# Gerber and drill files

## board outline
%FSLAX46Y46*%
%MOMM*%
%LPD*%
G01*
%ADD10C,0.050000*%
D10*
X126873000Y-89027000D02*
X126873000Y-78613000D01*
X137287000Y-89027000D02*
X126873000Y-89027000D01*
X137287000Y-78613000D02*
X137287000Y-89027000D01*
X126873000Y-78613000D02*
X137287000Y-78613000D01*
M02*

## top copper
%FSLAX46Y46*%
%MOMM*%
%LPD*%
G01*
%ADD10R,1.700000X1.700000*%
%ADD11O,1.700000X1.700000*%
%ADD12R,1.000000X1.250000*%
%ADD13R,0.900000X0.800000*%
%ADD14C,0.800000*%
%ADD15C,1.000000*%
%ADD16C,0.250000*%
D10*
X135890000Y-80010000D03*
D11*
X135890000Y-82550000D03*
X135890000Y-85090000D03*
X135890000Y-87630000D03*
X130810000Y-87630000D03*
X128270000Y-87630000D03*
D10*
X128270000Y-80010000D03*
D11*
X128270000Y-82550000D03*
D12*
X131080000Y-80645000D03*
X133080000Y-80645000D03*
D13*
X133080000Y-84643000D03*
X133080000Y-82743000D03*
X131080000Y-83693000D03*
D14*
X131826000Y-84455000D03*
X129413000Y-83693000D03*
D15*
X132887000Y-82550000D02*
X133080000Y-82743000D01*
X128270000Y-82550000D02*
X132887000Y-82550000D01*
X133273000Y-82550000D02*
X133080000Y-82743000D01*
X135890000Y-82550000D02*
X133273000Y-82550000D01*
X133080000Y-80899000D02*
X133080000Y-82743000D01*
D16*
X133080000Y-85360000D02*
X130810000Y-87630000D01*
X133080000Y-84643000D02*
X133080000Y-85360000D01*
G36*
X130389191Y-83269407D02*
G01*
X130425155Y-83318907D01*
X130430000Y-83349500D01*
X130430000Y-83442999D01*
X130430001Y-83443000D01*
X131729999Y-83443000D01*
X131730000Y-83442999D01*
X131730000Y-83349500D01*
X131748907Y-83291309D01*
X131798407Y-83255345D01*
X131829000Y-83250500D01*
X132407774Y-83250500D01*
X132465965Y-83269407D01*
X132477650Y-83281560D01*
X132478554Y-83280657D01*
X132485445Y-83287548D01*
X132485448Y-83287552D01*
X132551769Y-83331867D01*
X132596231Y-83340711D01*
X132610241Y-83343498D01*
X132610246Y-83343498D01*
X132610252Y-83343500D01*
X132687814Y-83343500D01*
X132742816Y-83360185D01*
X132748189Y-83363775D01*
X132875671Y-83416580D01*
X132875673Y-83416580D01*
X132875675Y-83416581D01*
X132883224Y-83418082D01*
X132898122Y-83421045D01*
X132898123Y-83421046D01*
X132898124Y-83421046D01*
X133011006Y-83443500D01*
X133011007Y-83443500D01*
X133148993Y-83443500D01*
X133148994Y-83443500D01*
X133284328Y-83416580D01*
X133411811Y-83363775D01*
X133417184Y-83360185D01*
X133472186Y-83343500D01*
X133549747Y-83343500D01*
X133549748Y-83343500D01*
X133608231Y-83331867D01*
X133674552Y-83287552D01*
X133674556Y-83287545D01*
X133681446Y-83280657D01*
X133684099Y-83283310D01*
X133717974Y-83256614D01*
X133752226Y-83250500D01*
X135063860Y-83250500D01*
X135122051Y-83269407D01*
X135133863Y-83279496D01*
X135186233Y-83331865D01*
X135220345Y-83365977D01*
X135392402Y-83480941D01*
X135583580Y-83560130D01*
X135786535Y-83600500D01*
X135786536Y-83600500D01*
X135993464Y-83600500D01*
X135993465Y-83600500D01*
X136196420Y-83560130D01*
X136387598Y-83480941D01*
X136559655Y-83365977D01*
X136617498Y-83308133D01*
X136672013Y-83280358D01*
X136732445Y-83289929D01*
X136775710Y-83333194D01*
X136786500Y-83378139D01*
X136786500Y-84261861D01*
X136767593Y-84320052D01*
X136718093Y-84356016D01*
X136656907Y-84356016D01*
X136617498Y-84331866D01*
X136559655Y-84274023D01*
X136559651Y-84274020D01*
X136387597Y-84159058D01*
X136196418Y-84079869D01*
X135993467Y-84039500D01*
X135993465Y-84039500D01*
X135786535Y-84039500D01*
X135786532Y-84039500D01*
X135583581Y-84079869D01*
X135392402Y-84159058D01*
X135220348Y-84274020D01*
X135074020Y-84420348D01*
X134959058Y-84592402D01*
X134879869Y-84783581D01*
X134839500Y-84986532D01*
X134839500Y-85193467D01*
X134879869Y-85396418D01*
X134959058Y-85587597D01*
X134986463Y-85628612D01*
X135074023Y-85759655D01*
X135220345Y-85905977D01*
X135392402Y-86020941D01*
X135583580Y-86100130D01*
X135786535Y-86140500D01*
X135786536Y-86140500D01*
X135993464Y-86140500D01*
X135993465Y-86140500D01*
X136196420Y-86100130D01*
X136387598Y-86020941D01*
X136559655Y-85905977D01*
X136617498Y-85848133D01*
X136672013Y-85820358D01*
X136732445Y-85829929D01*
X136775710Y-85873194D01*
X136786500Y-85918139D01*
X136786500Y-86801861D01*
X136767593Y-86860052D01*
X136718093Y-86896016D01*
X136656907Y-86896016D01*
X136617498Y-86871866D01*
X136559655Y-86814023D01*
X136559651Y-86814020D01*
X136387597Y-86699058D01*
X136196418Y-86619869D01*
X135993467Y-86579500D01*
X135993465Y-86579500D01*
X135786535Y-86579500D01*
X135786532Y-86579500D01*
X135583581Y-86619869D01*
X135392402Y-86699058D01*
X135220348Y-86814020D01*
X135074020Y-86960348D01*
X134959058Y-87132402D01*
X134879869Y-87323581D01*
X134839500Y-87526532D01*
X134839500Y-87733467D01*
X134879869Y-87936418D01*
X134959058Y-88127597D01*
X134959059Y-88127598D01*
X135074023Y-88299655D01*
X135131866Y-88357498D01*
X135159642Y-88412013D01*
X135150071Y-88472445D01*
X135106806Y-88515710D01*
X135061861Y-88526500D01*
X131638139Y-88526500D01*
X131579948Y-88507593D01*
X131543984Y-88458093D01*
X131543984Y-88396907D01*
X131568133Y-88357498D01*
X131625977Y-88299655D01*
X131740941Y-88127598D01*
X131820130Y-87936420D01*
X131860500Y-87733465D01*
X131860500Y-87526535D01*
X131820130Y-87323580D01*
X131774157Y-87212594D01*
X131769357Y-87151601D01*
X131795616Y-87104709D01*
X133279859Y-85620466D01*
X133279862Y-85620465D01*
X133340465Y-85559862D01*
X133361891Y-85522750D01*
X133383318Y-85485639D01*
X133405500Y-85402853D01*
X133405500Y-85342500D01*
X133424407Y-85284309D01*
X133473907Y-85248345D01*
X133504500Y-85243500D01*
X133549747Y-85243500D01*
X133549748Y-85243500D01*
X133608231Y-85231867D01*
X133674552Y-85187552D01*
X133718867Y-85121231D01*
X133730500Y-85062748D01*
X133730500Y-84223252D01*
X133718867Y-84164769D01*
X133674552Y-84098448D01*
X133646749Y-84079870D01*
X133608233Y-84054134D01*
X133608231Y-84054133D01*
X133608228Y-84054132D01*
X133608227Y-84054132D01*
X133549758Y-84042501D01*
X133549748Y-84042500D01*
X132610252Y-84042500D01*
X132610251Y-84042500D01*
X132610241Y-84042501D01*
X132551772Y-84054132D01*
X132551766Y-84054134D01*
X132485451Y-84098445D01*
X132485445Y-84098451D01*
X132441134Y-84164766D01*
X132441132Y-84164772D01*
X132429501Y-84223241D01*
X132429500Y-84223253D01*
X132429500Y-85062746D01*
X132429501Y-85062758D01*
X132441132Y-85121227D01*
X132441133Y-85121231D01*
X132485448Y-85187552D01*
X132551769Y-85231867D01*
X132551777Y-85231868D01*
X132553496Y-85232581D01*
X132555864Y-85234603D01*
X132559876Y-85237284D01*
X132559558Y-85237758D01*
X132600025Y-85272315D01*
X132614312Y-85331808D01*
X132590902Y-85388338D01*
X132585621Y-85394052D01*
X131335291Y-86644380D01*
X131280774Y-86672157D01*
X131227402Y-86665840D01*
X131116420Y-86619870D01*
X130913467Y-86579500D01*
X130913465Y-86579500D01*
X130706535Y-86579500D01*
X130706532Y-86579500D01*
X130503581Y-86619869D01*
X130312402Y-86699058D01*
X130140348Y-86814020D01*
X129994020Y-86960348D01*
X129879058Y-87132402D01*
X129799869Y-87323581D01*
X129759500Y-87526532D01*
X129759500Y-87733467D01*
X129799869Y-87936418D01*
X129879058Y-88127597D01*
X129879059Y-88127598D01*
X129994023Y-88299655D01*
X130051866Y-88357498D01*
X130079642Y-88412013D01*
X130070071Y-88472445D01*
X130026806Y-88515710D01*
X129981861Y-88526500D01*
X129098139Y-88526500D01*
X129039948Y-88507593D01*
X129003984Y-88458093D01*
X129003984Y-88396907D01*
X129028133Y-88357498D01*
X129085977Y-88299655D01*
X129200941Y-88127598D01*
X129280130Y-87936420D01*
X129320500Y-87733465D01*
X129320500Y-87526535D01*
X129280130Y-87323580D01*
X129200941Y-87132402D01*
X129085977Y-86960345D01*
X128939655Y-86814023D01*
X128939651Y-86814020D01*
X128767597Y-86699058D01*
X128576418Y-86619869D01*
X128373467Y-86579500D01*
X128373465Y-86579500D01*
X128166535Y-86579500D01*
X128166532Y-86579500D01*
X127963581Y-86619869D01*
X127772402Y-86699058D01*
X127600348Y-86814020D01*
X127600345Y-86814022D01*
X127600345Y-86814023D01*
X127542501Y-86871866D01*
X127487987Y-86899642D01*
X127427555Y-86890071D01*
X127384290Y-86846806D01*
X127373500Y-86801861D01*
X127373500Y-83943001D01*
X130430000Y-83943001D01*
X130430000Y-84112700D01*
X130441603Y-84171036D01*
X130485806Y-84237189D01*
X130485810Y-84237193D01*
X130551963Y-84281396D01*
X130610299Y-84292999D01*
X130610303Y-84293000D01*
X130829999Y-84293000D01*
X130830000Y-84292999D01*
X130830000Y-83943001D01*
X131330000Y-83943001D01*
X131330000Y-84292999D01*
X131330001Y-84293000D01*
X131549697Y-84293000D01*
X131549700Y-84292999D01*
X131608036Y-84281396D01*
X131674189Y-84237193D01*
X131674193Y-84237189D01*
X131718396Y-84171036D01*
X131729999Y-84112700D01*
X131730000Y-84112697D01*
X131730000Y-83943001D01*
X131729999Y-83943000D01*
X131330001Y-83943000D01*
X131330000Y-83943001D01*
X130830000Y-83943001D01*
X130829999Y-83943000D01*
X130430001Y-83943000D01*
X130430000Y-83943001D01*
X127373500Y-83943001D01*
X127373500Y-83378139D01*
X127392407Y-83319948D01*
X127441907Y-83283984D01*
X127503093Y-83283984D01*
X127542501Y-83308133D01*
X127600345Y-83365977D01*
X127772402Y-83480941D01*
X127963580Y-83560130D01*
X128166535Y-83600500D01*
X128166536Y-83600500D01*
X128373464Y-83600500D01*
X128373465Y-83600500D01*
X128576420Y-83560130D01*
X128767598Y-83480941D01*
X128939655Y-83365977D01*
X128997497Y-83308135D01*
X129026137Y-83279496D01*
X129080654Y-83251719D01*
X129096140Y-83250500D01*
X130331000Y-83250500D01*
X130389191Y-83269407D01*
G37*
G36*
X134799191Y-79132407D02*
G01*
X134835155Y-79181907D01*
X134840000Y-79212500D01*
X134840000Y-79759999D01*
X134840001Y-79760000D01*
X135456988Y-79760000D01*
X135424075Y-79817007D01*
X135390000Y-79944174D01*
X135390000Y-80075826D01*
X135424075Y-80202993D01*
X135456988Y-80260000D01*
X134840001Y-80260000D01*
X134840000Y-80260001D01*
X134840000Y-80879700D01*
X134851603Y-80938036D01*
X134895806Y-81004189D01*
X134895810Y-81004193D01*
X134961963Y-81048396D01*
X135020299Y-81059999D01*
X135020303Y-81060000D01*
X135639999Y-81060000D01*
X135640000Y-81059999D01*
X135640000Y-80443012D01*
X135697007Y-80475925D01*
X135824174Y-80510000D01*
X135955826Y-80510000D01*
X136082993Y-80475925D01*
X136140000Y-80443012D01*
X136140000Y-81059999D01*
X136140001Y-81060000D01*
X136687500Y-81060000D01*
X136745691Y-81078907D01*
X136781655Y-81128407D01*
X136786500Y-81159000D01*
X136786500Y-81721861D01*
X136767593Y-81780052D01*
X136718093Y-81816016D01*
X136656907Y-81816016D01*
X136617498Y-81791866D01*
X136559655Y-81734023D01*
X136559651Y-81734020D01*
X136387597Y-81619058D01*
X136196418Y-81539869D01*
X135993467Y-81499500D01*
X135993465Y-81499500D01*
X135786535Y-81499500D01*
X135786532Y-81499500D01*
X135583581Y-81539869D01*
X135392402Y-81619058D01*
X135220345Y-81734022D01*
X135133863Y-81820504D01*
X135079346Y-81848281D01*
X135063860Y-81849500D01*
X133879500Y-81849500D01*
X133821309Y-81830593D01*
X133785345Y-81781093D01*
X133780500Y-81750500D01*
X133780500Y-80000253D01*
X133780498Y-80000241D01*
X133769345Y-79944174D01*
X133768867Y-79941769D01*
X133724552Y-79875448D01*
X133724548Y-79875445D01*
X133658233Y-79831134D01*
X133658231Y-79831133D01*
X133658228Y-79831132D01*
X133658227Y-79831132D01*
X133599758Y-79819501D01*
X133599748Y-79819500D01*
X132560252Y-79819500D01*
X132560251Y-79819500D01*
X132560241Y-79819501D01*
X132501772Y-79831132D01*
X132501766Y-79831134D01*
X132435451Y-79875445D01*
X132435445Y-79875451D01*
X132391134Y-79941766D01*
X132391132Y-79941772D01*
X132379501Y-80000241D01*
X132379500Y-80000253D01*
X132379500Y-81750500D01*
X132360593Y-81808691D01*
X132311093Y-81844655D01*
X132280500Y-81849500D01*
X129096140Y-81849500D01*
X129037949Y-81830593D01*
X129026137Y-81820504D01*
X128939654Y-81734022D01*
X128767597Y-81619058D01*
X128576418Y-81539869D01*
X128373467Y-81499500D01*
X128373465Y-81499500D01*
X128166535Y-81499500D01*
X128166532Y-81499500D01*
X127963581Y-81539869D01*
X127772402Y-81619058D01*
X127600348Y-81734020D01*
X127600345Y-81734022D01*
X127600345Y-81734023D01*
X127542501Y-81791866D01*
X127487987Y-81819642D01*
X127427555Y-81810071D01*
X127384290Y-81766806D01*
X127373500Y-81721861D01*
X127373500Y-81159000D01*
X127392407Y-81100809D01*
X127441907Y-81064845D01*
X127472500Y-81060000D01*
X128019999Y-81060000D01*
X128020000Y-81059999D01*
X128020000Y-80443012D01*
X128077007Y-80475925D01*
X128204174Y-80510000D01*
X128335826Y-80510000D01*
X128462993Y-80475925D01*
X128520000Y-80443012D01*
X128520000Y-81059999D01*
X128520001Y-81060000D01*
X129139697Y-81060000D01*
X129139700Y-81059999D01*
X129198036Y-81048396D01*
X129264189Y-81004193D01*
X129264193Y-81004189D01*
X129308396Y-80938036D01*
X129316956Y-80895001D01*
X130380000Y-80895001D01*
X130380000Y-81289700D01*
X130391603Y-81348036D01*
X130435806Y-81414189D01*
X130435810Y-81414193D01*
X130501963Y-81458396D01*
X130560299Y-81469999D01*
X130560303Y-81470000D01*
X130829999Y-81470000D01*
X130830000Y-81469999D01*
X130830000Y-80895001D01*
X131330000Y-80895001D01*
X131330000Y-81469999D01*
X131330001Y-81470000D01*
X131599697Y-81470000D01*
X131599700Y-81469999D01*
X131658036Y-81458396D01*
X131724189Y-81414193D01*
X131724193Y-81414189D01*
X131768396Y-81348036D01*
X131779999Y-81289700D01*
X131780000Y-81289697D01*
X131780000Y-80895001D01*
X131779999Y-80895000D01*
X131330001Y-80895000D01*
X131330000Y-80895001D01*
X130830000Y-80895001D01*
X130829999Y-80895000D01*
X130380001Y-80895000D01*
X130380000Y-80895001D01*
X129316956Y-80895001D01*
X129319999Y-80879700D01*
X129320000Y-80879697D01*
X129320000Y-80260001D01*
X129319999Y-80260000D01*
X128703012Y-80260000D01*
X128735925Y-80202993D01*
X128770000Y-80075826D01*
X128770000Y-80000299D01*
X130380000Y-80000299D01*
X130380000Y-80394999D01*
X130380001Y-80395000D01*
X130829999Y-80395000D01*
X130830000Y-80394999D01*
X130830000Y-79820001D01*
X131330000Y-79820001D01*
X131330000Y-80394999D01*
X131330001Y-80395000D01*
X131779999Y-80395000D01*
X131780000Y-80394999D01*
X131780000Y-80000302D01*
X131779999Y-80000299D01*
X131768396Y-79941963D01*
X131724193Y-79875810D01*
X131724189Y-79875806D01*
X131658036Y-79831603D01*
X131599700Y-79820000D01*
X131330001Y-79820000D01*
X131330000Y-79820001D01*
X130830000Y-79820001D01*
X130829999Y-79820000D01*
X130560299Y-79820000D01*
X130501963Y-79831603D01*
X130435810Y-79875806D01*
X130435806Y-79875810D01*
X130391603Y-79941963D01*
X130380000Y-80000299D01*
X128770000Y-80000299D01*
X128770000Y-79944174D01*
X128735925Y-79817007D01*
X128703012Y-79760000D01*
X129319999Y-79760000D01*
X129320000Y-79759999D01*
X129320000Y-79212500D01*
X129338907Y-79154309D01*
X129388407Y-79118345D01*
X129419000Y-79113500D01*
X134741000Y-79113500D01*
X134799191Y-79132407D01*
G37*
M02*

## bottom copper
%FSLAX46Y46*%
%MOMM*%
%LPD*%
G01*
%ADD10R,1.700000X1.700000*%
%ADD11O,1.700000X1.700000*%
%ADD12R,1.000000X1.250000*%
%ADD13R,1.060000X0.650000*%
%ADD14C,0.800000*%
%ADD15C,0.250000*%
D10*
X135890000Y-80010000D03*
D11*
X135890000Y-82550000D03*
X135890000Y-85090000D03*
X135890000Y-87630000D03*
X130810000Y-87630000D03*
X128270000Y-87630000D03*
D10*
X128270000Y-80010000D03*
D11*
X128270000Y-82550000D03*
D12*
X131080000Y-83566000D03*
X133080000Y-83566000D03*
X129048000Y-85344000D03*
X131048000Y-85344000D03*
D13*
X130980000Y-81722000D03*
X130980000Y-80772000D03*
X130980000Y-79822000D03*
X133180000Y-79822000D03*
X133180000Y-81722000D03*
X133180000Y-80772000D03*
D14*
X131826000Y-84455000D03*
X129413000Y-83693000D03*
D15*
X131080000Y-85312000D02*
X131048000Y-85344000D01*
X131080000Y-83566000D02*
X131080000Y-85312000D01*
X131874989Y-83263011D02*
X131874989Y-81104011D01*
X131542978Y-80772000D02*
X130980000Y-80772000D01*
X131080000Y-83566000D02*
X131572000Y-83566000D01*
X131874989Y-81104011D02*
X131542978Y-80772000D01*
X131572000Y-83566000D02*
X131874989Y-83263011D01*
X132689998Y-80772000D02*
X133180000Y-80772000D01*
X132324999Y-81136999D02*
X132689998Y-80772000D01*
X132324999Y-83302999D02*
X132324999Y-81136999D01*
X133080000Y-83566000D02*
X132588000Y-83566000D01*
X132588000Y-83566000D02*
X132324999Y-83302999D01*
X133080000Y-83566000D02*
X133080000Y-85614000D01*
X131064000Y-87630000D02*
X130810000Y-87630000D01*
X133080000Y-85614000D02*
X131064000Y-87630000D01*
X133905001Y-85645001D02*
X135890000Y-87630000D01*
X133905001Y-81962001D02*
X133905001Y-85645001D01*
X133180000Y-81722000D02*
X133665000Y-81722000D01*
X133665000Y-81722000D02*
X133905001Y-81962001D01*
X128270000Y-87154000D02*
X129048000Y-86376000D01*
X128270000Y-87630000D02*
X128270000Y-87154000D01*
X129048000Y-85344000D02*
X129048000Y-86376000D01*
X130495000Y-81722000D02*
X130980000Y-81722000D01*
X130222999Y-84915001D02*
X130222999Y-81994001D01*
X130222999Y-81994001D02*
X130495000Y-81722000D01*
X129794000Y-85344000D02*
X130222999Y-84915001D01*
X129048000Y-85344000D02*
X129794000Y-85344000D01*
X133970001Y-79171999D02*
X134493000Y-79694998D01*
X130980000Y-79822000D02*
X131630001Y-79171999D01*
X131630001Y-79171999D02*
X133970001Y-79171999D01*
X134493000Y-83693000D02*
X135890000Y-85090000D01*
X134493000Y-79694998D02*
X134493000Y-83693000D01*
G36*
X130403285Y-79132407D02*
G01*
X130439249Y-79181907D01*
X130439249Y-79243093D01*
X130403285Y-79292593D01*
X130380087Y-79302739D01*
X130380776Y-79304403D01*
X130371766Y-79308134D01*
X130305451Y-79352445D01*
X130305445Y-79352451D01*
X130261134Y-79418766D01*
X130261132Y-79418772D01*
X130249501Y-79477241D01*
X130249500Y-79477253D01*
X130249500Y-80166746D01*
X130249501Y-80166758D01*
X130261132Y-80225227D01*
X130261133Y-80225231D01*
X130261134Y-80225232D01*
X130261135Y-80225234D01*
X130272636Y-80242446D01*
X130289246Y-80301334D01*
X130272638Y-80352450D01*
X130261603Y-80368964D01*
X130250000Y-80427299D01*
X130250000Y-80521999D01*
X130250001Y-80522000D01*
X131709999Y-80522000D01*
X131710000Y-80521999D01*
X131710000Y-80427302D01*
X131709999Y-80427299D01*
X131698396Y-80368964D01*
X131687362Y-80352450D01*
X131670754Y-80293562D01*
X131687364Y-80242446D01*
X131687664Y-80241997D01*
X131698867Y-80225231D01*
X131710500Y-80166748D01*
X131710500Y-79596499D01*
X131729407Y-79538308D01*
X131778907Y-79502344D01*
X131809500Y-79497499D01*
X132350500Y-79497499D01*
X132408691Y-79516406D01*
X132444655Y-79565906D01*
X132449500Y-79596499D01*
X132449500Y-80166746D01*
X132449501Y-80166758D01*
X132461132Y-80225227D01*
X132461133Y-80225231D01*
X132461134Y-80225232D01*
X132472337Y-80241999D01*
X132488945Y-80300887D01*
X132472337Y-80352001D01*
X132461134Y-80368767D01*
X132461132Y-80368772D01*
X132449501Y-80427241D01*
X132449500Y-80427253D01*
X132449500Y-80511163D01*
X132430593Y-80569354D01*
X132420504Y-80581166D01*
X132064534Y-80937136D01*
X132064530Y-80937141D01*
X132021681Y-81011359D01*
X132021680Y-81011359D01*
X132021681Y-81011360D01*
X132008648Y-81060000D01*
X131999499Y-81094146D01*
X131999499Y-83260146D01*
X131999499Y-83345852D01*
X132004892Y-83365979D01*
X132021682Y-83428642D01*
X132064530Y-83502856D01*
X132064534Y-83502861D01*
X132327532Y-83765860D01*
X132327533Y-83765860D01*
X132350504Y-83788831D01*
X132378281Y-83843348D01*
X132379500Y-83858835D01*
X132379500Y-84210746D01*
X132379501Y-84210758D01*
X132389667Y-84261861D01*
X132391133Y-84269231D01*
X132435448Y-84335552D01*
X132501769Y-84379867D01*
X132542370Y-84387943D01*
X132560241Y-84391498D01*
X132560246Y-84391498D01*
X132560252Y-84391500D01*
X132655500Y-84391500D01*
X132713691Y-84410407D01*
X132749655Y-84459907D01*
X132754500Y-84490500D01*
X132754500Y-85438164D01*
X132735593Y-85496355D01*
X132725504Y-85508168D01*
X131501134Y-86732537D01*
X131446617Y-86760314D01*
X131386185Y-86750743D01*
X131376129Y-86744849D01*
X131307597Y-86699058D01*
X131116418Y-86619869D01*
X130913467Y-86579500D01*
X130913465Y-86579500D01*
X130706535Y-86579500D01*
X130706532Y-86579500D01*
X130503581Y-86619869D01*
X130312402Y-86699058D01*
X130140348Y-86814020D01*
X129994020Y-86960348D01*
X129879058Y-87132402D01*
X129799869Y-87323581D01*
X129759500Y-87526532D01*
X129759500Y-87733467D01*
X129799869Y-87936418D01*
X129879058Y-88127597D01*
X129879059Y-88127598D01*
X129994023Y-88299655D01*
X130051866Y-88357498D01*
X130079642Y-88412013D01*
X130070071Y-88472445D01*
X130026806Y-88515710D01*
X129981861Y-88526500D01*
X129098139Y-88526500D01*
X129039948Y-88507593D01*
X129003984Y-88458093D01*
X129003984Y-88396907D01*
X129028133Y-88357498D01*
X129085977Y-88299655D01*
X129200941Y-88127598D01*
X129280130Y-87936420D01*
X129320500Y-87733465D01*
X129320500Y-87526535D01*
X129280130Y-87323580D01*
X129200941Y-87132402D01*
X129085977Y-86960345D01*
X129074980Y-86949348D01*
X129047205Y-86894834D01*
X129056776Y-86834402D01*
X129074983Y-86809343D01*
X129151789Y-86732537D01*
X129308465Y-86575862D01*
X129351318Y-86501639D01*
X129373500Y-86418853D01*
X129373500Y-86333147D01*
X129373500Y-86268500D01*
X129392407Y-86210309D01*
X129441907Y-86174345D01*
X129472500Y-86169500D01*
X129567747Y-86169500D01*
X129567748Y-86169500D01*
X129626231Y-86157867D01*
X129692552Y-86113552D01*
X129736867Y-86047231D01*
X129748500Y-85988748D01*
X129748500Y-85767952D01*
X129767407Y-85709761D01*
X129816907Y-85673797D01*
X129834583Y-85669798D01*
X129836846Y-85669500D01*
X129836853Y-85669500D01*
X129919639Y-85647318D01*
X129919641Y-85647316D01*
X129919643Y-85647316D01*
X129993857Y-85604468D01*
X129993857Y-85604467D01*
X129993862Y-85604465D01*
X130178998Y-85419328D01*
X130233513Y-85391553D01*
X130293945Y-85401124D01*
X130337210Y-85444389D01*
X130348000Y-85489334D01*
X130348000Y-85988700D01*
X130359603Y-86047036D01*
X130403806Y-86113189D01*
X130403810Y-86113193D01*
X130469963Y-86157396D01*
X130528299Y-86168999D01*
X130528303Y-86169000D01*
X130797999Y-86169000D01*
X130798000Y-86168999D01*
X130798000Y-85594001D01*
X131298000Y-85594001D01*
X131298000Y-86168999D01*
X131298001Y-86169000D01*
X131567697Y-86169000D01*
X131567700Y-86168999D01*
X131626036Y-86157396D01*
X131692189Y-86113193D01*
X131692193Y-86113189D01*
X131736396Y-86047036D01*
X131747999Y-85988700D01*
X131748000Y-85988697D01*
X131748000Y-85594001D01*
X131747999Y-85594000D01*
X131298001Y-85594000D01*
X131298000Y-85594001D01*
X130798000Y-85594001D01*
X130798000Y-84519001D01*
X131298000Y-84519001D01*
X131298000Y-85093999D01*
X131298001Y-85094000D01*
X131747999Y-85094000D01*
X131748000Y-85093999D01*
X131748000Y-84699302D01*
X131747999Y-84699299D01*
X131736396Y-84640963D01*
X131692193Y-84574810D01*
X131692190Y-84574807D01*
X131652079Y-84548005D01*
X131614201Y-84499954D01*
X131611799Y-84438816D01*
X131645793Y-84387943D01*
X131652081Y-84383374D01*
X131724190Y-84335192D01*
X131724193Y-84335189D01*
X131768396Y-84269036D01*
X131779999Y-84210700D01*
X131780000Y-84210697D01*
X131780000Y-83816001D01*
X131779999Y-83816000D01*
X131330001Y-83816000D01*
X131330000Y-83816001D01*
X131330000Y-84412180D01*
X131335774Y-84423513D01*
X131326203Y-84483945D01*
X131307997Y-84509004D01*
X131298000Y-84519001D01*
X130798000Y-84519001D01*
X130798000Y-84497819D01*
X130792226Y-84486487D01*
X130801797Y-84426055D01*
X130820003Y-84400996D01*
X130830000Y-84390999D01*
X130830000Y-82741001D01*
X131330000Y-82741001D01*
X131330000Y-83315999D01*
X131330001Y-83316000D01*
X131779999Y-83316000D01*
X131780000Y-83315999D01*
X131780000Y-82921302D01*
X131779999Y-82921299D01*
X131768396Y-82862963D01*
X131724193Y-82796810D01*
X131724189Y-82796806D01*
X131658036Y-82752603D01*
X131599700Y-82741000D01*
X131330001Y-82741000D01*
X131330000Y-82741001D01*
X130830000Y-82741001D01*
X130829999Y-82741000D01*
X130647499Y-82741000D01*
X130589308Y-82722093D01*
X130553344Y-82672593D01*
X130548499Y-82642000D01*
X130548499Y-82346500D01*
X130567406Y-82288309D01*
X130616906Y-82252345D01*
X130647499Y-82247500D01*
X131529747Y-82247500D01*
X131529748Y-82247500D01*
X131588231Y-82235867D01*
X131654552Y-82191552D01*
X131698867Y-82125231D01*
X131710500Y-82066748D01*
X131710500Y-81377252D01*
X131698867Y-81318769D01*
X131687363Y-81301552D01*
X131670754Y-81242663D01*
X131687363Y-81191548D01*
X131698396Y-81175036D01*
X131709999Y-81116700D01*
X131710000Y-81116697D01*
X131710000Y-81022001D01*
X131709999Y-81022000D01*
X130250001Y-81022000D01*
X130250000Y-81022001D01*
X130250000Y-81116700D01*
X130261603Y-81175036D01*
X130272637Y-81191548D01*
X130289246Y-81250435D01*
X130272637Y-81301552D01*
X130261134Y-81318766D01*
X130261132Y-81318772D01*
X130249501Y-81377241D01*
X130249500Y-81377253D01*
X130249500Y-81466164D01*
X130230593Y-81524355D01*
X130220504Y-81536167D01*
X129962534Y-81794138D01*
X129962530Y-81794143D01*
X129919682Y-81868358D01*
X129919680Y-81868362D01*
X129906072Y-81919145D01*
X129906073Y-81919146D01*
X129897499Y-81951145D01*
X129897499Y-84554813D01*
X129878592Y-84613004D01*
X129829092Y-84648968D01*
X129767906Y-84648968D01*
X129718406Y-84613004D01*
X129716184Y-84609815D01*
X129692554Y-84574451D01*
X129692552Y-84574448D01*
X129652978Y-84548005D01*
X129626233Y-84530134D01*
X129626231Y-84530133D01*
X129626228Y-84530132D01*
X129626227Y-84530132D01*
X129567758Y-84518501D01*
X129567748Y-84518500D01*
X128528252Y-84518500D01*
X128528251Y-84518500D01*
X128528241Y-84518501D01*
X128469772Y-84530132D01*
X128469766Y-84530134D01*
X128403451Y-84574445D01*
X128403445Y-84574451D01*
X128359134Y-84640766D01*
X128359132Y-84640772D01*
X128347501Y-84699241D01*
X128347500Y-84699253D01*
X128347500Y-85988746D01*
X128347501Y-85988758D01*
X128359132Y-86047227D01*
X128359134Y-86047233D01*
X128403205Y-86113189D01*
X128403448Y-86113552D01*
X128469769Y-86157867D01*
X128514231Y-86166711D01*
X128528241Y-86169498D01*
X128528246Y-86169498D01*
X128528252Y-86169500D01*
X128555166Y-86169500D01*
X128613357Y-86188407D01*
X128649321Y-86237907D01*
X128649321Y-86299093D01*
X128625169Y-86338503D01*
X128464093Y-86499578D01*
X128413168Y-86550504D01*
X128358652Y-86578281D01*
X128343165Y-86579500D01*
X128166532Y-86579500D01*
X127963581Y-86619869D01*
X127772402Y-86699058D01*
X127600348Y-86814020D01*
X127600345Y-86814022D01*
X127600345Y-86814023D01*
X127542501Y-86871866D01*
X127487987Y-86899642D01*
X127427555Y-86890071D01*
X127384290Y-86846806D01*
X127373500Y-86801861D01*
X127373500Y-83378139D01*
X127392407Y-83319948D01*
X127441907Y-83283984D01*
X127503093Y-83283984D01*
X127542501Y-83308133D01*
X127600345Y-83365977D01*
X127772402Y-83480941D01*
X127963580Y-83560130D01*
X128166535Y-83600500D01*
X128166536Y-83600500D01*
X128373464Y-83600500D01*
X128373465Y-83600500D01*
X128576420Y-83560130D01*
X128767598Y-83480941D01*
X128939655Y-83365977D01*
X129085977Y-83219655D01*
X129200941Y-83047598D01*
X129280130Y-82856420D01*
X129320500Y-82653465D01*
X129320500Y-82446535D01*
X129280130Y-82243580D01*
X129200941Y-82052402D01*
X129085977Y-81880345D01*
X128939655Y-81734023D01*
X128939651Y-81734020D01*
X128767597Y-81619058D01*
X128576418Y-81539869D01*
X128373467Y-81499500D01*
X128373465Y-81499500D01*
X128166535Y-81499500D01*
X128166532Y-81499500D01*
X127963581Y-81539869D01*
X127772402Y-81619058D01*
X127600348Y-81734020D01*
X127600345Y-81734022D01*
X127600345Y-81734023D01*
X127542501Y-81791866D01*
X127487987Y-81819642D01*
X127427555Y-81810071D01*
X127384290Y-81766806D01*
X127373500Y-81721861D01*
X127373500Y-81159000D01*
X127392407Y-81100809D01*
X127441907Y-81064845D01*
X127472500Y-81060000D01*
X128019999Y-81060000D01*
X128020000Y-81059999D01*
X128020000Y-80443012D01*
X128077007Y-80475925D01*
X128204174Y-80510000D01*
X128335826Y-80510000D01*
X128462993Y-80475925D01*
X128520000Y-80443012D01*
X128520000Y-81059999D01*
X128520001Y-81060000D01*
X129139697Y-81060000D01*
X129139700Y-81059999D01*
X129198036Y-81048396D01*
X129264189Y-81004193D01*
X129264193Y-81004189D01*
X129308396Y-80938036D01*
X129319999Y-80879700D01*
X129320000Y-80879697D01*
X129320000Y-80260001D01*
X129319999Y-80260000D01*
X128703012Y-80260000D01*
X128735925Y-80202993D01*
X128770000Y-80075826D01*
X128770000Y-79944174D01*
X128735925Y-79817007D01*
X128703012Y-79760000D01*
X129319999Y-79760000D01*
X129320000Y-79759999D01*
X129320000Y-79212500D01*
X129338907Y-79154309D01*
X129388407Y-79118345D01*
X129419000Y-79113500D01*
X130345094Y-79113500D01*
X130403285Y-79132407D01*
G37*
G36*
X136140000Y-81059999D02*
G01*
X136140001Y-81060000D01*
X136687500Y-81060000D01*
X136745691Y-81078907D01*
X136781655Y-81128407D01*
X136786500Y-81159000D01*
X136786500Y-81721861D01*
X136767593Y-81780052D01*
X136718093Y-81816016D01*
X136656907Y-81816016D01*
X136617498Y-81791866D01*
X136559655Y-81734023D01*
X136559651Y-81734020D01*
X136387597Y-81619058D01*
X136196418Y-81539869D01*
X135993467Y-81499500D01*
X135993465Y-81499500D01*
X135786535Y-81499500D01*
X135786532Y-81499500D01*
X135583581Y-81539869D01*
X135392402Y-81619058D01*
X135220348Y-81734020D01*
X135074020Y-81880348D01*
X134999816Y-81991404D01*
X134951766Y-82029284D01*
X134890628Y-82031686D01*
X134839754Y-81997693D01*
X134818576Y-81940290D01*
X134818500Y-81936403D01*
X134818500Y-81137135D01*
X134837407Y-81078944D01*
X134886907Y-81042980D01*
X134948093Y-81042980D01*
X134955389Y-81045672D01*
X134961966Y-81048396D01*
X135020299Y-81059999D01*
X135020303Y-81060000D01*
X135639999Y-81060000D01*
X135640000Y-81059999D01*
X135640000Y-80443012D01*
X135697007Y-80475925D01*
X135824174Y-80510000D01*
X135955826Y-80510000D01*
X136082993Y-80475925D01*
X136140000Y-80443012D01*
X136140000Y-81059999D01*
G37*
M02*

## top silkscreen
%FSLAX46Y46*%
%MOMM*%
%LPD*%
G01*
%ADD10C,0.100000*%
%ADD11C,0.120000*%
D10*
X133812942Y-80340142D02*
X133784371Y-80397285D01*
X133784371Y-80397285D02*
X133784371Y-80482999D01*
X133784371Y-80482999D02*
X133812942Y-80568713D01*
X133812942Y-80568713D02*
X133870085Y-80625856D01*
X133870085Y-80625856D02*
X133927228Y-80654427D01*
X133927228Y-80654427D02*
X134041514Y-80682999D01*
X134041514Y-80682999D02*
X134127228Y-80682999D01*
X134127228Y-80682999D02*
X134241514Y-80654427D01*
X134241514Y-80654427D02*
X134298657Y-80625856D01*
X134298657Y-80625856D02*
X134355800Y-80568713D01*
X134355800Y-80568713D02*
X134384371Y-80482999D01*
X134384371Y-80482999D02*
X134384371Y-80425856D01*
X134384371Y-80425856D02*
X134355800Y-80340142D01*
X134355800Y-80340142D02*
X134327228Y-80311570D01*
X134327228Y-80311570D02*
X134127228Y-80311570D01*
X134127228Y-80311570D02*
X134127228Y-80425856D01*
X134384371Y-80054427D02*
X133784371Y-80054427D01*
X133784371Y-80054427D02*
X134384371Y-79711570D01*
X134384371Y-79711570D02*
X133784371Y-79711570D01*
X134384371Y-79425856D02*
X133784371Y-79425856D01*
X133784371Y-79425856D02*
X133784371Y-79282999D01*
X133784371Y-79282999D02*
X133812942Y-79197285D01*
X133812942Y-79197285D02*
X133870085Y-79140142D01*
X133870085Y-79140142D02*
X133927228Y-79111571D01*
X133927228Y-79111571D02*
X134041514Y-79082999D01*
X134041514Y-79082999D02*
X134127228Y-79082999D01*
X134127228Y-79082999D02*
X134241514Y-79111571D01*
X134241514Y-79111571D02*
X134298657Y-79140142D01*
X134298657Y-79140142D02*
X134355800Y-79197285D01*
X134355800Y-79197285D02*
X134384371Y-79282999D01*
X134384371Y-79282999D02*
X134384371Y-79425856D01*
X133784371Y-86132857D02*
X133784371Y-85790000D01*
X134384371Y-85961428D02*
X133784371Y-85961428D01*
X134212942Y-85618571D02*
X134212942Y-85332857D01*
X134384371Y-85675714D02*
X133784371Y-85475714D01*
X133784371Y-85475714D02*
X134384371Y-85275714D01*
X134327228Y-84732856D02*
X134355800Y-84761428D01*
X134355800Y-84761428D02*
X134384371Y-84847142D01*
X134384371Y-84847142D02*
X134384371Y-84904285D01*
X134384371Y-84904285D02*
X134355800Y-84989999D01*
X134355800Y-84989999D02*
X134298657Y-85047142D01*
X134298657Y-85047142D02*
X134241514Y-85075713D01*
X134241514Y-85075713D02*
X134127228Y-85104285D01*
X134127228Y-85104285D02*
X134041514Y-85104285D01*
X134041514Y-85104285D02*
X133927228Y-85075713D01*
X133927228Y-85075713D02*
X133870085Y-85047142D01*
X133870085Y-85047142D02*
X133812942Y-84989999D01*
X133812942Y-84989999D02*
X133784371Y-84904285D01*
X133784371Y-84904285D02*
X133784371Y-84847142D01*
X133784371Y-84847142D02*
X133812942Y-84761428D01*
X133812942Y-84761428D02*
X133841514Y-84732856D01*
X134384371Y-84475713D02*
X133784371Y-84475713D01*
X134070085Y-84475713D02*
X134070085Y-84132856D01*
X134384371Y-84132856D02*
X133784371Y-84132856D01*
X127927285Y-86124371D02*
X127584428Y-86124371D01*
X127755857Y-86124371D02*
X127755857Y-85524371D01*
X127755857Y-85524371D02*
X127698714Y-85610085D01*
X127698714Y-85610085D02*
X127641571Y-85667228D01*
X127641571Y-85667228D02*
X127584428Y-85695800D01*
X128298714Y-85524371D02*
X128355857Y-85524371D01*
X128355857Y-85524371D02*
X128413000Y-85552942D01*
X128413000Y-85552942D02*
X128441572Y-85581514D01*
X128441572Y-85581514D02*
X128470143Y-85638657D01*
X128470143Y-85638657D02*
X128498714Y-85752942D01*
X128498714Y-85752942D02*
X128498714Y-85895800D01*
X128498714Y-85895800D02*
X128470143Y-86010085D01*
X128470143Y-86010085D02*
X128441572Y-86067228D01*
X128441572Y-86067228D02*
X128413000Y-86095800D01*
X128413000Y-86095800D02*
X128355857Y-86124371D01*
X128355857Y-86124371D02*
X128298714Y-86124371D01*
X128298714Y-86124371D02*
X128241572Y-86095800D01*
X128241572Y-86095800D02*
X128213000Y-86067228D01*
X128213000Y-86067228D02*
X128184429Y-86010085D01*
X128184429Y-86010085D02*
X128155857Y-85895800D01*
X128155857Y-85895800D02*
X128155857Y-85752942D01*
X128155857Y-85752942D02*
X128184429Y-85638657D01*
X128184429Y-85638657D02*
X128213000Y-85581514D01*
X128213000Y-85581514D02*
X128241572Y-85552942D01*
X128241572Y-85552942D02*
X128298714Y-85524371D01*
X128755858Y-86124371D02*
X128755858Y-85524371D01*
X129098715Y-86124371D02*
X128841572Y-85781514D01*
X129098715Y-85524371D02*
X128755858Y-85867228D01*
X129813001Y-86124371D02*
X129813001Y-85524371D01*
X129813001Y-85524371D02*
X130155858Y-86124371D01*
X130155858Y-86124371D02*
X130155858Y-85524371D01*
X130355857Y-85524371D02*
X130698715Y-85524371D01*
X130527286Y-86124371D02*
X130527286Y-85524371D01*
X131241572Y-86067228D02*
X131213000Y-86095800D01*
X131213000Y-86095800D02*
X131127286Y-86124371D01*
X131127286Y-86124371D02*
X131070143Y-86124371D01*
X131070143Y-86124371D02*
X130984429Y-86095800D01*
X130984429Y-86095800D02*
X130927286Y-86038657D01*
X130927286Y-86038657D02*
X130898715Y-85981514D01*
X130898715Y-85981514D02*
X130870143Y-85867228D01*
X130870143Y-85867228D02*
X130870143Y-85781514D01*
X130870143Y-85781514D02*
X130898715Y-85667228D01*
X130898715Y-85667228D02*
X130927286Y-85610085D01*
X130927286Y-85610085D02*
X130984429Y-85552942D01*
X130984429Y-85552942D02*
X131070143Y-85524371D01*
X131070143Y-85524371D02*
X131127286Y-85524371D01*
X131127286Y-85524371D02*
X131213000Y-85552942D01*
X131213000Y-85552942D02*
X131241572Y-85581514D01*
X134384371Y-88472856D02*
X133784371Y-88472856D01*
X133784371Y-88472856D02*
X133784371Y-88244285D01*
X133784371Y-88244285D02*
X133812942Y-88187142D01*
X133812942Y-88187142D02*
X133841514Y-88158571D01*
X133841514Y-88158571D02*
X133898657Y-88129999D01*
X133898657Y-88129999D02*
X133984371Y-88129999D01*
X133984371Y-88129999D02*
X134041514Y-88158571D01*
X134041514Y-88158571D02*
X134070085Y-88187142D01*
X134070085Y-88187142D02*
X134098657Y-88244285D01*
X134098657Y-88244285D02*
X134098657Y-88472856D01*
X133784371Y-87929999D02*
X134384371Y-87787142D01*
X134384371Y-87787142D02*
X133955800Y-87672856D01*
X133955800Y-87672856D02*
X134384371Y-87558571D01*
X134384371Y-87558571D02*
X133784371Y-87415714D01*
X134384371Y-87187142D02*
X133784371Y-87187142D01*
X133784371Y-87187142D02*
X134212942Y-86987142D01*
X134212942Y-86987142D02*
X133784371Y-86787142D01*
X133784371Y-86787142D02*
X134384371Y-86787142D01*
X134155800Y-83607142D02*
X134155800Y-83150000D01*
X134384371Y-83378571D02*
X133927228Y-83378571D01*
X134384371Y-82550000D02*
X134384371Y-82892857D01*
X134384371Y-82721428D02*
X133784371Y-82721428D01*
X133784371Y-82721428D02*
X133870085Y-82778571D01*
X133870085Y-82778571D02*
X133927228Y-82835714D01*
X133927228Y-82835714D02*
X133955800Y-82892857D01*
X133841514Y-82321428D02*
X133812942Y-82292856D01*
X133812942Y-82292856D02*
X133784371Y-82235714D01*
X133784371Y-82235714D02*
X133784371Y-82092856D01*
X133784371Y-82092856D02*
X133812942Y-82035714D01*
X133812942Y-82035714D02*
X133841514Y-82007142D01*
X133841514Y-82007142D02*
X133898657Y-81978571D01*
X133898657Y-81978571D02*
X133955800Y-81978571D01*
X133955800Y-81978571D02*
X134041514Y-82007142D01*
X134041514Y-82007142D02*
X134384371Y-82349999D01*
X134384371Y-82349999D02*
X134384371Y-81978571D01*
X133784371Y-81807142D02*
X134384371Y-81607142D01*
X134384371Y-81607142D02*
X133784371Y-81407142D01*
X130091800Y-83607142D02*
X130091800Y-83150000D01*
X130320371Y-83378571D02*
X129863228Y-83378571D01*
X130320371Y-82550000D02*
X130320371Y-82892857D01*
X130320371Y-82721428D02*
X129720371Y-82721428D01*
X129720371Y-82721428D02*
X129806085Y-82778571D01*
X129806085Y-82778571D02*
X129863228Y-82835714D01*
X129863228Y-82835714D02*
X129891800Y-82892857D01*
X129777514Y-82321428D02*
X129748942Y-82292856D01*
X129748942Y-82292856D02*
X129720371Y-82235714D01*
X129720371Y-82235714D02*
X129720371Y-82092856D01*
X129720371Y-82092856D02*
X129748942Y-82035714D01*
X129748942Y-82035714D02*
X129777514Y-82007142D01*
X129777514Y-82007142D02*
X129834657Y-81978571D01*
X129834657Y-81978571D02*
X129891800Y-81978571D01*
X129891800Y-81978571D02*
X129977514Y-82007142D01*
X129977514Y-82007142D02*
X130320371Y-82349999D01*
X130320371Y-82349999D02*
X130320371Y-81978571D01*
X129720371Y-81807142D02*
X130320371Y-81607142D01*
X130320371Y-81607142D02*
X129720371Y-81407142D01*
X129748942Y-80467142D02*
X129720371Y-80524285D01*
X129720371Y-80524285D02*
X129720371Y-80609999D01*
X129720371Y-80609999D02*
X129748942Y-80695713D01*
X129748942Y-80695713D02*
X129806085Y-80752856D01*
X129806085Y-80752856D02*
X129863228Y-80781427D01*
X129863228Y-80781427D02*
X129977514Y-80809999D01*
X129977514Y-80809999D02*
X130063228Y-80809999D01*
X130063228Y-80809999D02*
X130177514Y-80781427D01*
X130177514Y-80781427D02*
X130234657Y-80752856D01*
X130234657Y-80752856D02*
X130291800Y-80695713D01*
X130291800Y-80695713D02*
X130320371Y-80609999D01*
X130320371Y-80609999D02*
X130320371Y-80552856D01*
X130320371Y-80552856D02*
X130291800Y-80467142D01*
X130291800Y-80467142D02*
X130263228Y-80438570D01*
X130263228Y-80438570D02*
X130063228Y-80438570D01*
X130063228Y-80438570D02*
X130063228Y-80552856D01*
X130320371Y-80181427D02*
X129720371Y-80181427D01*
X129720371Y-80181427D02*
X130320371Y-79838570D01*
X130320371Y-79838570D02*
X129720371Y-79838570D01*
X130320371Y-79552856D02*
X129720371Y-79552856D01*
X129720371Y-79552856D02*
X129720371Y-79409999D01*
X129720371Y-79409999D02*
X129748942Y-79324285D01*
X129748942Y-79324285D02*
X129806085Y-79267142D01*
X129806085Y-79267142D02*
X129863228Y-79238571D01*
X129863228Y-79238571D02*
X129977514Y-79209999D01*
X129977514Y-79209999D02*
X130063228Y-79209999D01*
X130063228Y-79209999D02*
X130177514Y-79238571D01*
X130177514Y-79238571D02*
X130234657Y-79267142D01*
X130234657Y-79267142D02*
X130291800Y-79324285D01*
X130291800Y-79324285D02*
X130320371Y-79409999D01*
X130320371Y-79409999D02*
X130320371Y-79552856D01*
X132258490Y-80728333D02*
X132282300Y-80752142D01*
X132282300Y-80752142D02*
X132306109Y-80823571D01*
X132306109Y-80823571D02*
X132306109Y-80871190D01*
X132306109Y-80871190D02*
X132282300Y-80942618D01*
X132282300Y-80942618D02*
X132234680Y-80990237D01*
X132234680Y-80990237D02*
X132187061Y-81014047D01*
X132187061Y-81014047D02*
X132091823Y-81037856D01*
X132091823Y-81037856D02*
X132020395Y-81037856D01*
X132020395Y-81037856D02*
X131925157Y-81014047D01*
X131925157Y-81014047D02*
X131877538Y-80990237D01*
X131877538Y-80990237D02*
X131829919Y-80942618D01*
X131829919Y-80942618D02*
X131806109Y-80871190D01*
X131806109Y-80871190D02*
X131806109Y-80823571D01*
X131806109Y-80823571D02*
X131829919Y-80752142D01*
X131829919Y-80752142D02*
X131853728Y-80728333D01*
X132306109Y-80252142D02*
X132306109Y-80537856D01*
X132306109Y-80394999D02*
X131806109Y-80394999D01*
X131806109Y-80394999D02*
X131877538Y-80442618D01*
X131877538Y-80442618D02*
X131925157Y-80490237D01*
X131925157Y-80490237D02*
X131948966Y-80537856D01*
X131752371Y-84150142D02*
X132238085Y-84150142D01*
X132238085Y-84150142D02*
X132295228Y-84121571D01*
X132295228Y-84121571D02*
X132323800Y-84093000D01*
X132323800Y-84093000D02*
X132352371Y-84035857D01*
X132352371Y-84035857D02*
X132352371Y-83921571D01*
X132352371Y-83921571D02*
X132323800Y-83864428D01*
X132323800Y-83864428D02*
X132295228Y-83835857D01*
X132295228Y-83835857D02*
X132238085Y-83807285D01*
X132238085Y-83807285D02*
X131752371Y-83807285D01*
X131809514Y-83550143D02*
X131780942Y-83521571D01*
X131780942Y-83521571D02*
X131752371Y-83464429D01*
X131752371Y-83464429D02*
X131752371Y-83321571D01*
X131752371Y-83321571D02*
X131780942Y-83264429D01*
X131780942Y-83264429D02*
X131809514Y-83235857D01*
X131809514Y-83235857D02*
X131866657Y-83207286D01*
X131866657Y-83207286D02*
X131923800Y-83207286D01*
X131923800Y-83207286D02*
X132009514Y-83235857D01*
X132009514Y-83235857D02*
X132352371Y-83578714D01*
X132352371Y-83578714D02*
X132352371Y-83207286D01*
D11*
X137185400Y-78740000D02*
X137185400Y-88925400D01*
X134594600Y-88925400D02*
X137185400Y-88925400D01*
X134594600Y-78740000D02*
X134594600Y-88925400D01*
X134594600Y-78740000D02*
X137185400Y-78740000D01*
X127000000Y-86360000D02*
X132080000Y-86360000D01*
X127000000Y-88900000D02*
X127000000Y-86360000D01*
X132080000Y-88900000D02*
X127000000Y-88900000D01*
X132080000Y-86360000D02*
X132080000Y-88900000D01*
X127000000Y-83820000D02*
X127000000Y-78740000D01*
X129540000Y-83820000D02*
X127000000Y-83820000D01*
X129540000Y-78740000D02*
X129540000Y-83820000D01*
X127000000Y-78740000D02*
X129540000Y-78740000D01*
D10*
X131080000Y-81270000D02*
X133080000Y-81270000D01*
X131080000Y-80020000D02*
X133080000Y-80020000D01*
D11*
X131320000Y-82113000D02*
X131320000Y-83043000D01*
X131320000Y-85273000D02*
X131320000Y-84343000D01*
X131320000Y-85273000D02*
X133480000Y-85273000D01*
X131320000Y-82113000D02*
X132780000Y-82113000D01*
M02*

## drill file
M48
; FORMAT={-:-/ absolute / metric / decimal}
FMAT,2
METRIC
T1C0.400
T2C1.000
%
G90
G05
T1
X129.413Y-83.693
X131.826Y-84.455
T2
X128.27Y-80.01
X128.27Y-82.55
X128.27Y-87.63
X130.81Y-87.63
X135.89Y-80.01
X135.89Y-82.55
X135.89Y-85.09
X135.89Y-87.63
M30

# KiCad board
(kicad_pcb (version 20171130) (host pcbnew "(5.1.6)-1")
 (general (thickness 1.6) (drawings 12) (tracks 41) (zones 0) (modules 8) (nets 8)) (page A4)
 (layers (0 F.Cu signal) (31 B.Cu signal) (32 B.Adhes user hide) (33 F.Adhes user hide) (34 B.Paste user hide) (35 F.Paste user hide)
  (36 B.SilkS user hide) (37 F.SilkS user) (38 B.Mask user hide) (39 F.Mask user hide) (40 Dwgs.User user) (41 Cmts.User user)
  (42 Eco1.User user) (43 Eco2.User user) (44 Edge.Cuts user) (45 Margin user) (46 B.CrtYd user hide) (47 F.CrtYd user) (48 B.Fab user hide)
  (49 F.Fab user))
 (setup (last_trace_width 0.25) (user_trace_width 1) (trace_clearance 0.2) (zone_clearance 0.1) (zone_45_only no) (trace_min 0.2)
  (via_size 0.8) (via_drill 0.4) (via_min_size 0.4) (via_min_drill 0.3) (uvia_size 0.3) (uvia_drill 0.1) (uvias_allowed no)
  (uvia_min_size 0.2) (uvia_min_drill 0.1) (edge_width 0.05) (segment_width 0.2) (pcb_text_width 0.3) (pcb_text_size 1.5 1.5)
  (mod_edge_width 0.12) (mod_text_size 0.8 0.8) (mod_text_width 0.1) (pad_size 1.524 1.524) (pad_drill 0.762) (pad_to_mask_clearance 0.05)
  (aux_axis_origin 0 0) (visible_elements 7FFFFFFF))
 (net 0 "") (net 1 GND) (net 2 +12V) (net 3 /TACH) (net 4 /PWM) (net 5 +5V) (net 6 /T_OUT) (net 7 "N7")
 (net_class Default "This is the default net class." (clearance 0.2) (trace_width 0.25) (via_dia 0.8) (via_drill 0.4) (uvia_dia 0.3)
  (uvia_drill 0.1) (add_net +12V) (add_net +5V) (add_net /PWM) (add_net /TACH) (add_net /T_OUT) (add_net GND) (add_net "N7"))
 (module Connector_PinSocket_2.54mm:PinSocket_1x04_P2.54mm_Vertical (layer F.Cu) (at 135.89 80.01)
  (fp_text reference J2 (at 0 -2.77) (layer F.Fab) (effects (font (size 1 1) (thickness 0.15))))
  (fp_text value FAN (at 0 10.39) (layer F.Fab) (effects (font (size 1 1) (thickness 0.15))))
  (fp_line (start 1.2954 -1.27) (end 1.2954 8.9154) (layer F.SilkS) (width 0.12))
  (fp_line (start -1.2954 8.9154) (end 1.2954 8.9154) (layer F.SilkS) (width 0.12))
  (fp_line (start -1.2954 -1.27) (end -1.2954 8.9154) (layer F.SilkS) (width 0.12))
  (fp_line (start -1.2954 -1.27) (end 1.2954 -1.27) (layer F.SilkS) (width 0.12))
  (pad 1 thru_hole rect (at 0 0) (size 1.7 1.7) (drill 1) (layers *.Cu *.Mask) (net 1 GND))
  (pad 2 thru_hole oval (at 0 2.54) (size 1.7 1.7) (drill 1) (layers *.Cu *.Mask) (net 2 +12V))
  (pad 3 thru_hole oval (at 0 5.08) (size 1.7 1.7) (drill 1) (layers *.Cu *.Mask) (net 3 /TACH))
  (pad 4 thru_hole oval (at 0 7.62) (size 1.7 1.7) (drill 1) (layers *.Cu *.Mask) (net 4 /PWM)))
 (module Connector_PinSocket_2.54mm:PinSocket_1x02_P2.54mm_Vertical (layer F.Cu) (at 130.81 87.63 270)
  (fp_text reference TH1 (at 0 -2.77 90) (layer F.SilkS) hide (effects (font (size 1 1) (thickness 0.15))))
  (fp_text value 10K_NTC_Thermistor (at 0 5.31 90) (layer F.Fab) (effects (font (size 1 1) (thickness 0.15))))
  (fp_line (start -1.27 3.81) (end -1.27 -1.27) (layer F.SilkS) (width 0.12))
  (fp_line (start 1.27 3.81) (end -1.27 3.81) (layer F.SilkS) (width 0.12))
  (fp_line (start 1.27 -1.27) (end 1.27 3.81) (layer F.SilkS) (width 0.12))
  (fp_line (start -1.27 -1.27) (end 1.27 -1.27) (layer F.SilkS) (width 0.12))
  (pad 1 thru_hole oval (at 0 0 270) (size 1.7 1.7) (drill 1) (layers *.Cu *.Mask) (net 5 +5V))
  (pad 2 thru_hole oval (at 0 2.54 270) (size 1.7 1.7) (drill 1) (layers *.Cu *.Mask) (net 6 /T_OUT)))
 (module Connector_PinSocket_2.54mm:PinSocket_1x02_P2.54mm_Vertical (layer F.Cu) (at 128.27 80.01)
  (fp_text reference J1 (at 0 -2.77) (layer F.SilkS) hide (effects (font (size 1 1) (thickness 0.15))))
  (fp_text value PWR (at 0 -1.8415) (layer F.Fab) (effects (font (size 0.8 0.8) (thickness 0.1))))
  (fp_line (start -1.27 3.81) (end -1.27 -1.27) (layer F.SilkS) (width 0.12))
  (fp_line (start 1.27 3.81) (end -1.27 3.81) (layer F.SilkS) (width 0.12))
  (fp_line (start 1.27 -1.27) (end 1.27 3.81) (layer F.SilkS) (width 0.12))
  (fp_line (start -1.27 -1.27) (end 1.27 -1.27) (layer F.SilkS) (width 0.12))
  (pad 1 thru_hole rect (at 0 0) (size 1.7 1.7) (drill 1) (layers *.Cu *.Mask) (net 1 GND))
  (pad 2 thru_hole oval (at 0 2.54) (size 1.7 1.7) (drill 1) (layers *.Cu *.Mask) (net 2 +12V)))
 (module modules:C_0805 (layer F.Cu) (at 132.08 80.645)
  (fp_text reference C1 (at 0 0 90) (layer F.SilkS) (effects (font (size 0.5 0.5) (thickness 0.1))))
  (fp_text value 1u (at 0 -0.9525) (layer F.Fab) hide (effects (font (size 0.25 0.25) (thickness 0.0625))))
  (fp_line (start -1 0.625) (end 1 0.625) (layer F.SilkS) (width 0.1))
  (fp_line (start -1 -0.625) (end 1 -0.625) (layer F.SilkS) (width 0.1))
  (pad 1 smd rect (at -1 0) (size 1 1.25) (layers F.Cu F.Paste F.Mask) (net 1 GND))
  (pad 2 smd rect (at 1 0) (size 1 1.25) (layers F.Cu F.Paste F.Mask) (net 2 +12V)))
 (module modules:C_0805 (layer B.Cu) (at 132.08 83.566 180)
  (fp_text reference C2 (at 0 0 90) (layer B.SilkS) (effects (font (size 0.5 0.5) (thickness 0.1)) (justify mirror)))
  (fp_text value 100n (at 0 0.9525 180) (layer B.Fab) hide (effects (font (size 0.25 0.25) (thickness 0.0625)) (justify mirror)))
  (pad 2 smd rect (at 1 0 180) (size 1 1.25) (layers B.Cu B.Paste B.Mask) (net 1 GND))
  (pad 1 smd rect (at -1 0 180) (size 1 1.25) (layers B.Cu B.Paste B.Mask) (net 5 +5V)))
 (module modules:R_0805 (layer B.Cu) (at 130.048 85.344)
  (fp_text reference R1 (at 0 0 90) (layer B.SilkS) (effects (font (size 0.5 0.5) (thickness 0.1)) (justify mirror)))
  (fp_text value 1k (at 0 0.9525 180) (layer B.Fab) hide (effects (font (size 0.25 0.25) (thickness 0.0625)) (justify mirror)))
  (pad 1 smd rect (at -1 0) (size 1 1.25) (layers B.Cu B.Paste B.Mask) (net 6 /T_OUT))
  (pad 2 smd rect (at 1 0) (size 1 1.25) (layers B.Cu B.Paste B.Mask) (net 1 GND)))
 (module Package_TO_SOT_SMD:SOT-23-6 (layer B.Cu) (at 132.08 80.772)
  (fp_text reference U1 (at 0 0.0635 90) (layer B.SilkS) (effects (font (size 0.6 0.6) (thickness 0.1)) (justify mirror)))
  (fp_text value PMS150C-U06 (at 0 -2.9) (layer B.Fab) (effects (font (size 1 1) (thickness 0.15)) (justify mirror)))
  (pad 1 smd rect (at -1.1 0.95) (size 1.06 0.65) (layers B.Cu B.Paste B.Mask) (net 6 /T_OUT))
  (pad 2 smd rect (at -1.1 0) (size 1.06 0.65) (layers B.Cu B.Paste B.Mask) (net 1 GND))
  (pad 3 smd rect (at -1.1 -0.95) (size 1.06 0.65) (layers B.Cu B.Paste B.Mask) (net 3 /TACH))
  (pad 4 smd rect (at 1.1 -0.95) (size 1.06 0.65) (layers B.Cu B.Paste B.Mask) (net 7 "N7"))
  (pad 6 smd rect (at 1.1 0.95) (size 1.06 0.65) (layers B.Cu B.Paste B.Mask) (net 4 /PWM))
  (pad 5 smd rect (at 1.1 0) (size 1.06 0.65) (layers B.Cu B.Paste B.Mask) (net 5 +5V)))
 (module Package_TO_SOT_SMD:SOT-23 (layer F.Cu) (at 132.08 83.693 180)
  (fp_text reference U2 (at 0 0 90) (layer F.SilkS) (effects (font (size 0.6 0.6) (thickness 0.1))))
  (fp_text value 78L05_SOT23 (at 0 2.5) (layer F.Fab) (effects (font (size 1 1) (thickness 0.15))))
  (fp_line (start 0.76 1.58) (end 0.76 0.65) (layer F.SilkS) (width 0.12))
  (fp_line (start 0.76 -1.58) (end 0.76 -0.65) (layer F.SilkS) (width 0.12))
  (fp_line (start 0.76 -1.58) (end -1.4 -1.58) (layer F.SilkS) (width 0.12))
  (fp_line (start 0.76 1.58) (end -0.7 1.58) (layer F.SilkS) (width 0.12))
  (pad 1 smd rect (at -1 -0.95 180) (size 0.9 0.8) (layers F.Cu F.Paste F.Mask) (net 5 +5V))
  (pad 2 smd rect (at -1 0.95 180) (size 0.9 0.8) (layers F.Cu F.Paste F.Mask) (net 2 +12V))
  (pad 3 smd rect (at 1 0 180) (size 0.9 0.8) (layers F.Cu F.Paste F.Mask) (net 1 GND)))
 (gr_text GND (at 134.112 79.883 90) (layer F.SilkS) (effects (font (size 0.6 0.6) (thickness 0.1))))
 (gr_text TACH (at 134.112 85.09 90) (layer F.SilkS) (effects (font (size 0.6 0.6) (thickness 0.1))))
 (gr_line (start 126.873 89.027) (end 126.873 78.613) (layer Edge.Cuts) (width 0.05))
 (gr_line (start 137.287 89.027) (end 126.873 89.027) (layer Edge.Cuts) (width 0.05))
 (gr_line (start 137.287 78.613) (end 137.287 89.027) (layer Edge.Cuts) (width 0.05))
 (gr_line (start 126.873 78.613) (end 137.287 78.613) (layer Edge.Cuts) (width 0.05))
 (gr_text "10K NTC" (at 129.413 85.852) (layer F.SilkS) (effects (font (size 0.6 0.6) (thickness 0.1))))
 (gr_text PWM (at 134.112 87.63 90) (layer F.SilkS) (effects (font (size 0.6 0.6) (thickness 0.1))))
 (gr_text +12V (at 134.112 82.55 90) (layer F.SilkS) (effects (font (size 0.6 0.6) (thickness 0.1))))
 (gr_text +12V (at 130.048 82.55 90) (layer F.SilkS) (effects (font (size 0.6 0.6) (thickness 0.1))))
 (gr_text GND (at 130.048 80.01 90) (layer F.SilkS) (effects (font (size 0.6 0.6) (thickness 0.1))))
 (segment (start 131.08 85.312) (end 131.048 85.344) (width 0.25) (layer B.Cu) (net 1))
 (segment (start 131.08 83.566) (end 131.08 85.312) (width 0.25) (layer B.Cu) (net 1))
 (via (at 131.826 84.455) (size 0.8) (drill 0.4) (layers F.Cu B.Cu) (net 1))
 (segment (start 131.874989 83.263011) (end 131.874989 81.104011) (width 0.25) (layer B.Cu) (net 1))
 (segment (start 131.542978 80.772) (end 130.98 80.772) (width 0.25) (layer B.Cu) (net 1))
 (segment (start 131.08 83.566) (end 131.572 83.566) (width 0.25) (layer B.Cu) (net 1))
 (segment (start 131.874989 81.104011) (end 131.542978 80.772) (width 0.25) (layer B.Cu) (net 1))
 (segment (start 131.572 83.566) (end 131.874989 83.263011) (width 0.25) (layer B.Cu) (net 1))
 (via (at 129.413 83.693) (size 0.8) (drill 0.4) (layers F.Cu B.Cu) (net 1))
 (segment (start 132.887 82.55) (end 133.08 82.743) (width 1) (layer F.Cu) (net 2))
 (segment (start 128.27 82.55) (end 132.887 82.55) (width 1) (layer F.Cu) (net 2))
 (segment (start 133.273 82.55) (end 133.08 82.743) (width 1) (layer F.Cu) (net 2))
 (segment (start 135.89 82.55) (end 133.273 82.55) (width 1) (layer F.Cu) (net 2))
 (segment (start 133.08 80.899) (end 133.08 82.743) (width 1) (layer F.Cu) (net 2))
 (segment (start 133.08 85.36) (end 130.81 87.63) (width 0.25) (layer F.Cu) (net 5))
 (segment (start 133.08 84.643) (end 133.08 85.36) (width 0.25) (layer F.Cu) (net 5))
 (segment (start 132.689998 80.772) (end 133.18 80.772) (width 0.25) (layer B.Cu) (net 5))
 (segment (start 132.324999 81.136999) (end 132.689998 80.772) (width 0.25) (layer B.Cu) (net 5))
 (segment (start 132.324999 83.302999) (end 132.324999 81.136999) (width 0.25) (layer B.Cu) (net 5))
 (segment (start 133.08 83.566) (end 132.588 83.566) (width 0.25) (layer B.Cu) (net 5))
 (segment (start 132.588 83.566) (end 132.324999 83.302999) (width 0.25) (layer B.Cu) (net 5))
 (segment (start 133.08 83.566) (end 133.08 85.614) (width 0.25) (layer B.Cu) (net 5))
 (segment (start 131.064 87.63) (end 130.81 87.63) (width 0.25) (layer B.Cu) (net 5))
 (segment (start 133.08 85.614) (end 131.064 87.63) (width 0.25) (layer B.Cu) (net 5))
 (segment (start 133.905001 85.645001) (end 135.89 87.63) (width 0.25) (layer B.Cu) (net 4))
 (segment (start 133.905001 81.962001) (end 133.905001 85.645001) (width 0.25) (layer B.Cu) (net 4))
 (segment (start 133.18 81.722) (end 133.665 81.722) (width 0.25) (layer B.Cu) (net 4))
 (segment (start 133.665 81.722) (end 133.905001 81.962001) (width 0.25) (layer B.Cu) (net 4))
 (segment (start 128.27 87.154) (end 129.048 86.376) (width 0.25) (layer B.Cu) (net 6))
 (segment (start 128.27 87.63) (end 128.27 87.154) (width 0.25) (layer B.Cu) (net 6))
 (segment (start 129.048 85.344) (end 129.048 86.376) (width 0.25) (layer B.Cu) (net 6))
 (segment (start 130.495 81.722) (end 130.98 81.722) (width 0.25) (layer B.Cu) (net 6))
 (segment (start 130.222999 84.915001) (end 130.222999 81.994001) (width 0.25) (layer B.Cu) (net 6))
 (segment (start 130.222999 81.994001) (end 130.495 81.722) (width 0.25) (layer B.Cu) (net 6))
 (segment (start 129.794 85.344) (end 130.222999 84.915001) (width 0.25) (layer B.Cu) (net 6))
 (segment (start 129.048 85.344) (end 129.794 85.344) (width 0.25) (layer B.Cu) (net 6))
 (segment (start 133.970001 79.171999) (end 134.493 79.694998) (width 0.25) (layer B.Cu) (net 3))
 (segment (start 130.98 79.822) (end 131.630001 79.171999) (width 0.25) (layer B.Cu) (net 3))
 (segment (start 131.630001 79.171999) (end 133.970001 79.171999) (width 0.25) (layer B.Cu) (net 3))
 (segment (start 134.493 83.693) (end 135.89 85.09) (width 0.25) (layer B.Cu) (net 3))
 (segment (start 134.493 79.694998) (end 134.493 83.693) (width 0.25) (layer B.Cu) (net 3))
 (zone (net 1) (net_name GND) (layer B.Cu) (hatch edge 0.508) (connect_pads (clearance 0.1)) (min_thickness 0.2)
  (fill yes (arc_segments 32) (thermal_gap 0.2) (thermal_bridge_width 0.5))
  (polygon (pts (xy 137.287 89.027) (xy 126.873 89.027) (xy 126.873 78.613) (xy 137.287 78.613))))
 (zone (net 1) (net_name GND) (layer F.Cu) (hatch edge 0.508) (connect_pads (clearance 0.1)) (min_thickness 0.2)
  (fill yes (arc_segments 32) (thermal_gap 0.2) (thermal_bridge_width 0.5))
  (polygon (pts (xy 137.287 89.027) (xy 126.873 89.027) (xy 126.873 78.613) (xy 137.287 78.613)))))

